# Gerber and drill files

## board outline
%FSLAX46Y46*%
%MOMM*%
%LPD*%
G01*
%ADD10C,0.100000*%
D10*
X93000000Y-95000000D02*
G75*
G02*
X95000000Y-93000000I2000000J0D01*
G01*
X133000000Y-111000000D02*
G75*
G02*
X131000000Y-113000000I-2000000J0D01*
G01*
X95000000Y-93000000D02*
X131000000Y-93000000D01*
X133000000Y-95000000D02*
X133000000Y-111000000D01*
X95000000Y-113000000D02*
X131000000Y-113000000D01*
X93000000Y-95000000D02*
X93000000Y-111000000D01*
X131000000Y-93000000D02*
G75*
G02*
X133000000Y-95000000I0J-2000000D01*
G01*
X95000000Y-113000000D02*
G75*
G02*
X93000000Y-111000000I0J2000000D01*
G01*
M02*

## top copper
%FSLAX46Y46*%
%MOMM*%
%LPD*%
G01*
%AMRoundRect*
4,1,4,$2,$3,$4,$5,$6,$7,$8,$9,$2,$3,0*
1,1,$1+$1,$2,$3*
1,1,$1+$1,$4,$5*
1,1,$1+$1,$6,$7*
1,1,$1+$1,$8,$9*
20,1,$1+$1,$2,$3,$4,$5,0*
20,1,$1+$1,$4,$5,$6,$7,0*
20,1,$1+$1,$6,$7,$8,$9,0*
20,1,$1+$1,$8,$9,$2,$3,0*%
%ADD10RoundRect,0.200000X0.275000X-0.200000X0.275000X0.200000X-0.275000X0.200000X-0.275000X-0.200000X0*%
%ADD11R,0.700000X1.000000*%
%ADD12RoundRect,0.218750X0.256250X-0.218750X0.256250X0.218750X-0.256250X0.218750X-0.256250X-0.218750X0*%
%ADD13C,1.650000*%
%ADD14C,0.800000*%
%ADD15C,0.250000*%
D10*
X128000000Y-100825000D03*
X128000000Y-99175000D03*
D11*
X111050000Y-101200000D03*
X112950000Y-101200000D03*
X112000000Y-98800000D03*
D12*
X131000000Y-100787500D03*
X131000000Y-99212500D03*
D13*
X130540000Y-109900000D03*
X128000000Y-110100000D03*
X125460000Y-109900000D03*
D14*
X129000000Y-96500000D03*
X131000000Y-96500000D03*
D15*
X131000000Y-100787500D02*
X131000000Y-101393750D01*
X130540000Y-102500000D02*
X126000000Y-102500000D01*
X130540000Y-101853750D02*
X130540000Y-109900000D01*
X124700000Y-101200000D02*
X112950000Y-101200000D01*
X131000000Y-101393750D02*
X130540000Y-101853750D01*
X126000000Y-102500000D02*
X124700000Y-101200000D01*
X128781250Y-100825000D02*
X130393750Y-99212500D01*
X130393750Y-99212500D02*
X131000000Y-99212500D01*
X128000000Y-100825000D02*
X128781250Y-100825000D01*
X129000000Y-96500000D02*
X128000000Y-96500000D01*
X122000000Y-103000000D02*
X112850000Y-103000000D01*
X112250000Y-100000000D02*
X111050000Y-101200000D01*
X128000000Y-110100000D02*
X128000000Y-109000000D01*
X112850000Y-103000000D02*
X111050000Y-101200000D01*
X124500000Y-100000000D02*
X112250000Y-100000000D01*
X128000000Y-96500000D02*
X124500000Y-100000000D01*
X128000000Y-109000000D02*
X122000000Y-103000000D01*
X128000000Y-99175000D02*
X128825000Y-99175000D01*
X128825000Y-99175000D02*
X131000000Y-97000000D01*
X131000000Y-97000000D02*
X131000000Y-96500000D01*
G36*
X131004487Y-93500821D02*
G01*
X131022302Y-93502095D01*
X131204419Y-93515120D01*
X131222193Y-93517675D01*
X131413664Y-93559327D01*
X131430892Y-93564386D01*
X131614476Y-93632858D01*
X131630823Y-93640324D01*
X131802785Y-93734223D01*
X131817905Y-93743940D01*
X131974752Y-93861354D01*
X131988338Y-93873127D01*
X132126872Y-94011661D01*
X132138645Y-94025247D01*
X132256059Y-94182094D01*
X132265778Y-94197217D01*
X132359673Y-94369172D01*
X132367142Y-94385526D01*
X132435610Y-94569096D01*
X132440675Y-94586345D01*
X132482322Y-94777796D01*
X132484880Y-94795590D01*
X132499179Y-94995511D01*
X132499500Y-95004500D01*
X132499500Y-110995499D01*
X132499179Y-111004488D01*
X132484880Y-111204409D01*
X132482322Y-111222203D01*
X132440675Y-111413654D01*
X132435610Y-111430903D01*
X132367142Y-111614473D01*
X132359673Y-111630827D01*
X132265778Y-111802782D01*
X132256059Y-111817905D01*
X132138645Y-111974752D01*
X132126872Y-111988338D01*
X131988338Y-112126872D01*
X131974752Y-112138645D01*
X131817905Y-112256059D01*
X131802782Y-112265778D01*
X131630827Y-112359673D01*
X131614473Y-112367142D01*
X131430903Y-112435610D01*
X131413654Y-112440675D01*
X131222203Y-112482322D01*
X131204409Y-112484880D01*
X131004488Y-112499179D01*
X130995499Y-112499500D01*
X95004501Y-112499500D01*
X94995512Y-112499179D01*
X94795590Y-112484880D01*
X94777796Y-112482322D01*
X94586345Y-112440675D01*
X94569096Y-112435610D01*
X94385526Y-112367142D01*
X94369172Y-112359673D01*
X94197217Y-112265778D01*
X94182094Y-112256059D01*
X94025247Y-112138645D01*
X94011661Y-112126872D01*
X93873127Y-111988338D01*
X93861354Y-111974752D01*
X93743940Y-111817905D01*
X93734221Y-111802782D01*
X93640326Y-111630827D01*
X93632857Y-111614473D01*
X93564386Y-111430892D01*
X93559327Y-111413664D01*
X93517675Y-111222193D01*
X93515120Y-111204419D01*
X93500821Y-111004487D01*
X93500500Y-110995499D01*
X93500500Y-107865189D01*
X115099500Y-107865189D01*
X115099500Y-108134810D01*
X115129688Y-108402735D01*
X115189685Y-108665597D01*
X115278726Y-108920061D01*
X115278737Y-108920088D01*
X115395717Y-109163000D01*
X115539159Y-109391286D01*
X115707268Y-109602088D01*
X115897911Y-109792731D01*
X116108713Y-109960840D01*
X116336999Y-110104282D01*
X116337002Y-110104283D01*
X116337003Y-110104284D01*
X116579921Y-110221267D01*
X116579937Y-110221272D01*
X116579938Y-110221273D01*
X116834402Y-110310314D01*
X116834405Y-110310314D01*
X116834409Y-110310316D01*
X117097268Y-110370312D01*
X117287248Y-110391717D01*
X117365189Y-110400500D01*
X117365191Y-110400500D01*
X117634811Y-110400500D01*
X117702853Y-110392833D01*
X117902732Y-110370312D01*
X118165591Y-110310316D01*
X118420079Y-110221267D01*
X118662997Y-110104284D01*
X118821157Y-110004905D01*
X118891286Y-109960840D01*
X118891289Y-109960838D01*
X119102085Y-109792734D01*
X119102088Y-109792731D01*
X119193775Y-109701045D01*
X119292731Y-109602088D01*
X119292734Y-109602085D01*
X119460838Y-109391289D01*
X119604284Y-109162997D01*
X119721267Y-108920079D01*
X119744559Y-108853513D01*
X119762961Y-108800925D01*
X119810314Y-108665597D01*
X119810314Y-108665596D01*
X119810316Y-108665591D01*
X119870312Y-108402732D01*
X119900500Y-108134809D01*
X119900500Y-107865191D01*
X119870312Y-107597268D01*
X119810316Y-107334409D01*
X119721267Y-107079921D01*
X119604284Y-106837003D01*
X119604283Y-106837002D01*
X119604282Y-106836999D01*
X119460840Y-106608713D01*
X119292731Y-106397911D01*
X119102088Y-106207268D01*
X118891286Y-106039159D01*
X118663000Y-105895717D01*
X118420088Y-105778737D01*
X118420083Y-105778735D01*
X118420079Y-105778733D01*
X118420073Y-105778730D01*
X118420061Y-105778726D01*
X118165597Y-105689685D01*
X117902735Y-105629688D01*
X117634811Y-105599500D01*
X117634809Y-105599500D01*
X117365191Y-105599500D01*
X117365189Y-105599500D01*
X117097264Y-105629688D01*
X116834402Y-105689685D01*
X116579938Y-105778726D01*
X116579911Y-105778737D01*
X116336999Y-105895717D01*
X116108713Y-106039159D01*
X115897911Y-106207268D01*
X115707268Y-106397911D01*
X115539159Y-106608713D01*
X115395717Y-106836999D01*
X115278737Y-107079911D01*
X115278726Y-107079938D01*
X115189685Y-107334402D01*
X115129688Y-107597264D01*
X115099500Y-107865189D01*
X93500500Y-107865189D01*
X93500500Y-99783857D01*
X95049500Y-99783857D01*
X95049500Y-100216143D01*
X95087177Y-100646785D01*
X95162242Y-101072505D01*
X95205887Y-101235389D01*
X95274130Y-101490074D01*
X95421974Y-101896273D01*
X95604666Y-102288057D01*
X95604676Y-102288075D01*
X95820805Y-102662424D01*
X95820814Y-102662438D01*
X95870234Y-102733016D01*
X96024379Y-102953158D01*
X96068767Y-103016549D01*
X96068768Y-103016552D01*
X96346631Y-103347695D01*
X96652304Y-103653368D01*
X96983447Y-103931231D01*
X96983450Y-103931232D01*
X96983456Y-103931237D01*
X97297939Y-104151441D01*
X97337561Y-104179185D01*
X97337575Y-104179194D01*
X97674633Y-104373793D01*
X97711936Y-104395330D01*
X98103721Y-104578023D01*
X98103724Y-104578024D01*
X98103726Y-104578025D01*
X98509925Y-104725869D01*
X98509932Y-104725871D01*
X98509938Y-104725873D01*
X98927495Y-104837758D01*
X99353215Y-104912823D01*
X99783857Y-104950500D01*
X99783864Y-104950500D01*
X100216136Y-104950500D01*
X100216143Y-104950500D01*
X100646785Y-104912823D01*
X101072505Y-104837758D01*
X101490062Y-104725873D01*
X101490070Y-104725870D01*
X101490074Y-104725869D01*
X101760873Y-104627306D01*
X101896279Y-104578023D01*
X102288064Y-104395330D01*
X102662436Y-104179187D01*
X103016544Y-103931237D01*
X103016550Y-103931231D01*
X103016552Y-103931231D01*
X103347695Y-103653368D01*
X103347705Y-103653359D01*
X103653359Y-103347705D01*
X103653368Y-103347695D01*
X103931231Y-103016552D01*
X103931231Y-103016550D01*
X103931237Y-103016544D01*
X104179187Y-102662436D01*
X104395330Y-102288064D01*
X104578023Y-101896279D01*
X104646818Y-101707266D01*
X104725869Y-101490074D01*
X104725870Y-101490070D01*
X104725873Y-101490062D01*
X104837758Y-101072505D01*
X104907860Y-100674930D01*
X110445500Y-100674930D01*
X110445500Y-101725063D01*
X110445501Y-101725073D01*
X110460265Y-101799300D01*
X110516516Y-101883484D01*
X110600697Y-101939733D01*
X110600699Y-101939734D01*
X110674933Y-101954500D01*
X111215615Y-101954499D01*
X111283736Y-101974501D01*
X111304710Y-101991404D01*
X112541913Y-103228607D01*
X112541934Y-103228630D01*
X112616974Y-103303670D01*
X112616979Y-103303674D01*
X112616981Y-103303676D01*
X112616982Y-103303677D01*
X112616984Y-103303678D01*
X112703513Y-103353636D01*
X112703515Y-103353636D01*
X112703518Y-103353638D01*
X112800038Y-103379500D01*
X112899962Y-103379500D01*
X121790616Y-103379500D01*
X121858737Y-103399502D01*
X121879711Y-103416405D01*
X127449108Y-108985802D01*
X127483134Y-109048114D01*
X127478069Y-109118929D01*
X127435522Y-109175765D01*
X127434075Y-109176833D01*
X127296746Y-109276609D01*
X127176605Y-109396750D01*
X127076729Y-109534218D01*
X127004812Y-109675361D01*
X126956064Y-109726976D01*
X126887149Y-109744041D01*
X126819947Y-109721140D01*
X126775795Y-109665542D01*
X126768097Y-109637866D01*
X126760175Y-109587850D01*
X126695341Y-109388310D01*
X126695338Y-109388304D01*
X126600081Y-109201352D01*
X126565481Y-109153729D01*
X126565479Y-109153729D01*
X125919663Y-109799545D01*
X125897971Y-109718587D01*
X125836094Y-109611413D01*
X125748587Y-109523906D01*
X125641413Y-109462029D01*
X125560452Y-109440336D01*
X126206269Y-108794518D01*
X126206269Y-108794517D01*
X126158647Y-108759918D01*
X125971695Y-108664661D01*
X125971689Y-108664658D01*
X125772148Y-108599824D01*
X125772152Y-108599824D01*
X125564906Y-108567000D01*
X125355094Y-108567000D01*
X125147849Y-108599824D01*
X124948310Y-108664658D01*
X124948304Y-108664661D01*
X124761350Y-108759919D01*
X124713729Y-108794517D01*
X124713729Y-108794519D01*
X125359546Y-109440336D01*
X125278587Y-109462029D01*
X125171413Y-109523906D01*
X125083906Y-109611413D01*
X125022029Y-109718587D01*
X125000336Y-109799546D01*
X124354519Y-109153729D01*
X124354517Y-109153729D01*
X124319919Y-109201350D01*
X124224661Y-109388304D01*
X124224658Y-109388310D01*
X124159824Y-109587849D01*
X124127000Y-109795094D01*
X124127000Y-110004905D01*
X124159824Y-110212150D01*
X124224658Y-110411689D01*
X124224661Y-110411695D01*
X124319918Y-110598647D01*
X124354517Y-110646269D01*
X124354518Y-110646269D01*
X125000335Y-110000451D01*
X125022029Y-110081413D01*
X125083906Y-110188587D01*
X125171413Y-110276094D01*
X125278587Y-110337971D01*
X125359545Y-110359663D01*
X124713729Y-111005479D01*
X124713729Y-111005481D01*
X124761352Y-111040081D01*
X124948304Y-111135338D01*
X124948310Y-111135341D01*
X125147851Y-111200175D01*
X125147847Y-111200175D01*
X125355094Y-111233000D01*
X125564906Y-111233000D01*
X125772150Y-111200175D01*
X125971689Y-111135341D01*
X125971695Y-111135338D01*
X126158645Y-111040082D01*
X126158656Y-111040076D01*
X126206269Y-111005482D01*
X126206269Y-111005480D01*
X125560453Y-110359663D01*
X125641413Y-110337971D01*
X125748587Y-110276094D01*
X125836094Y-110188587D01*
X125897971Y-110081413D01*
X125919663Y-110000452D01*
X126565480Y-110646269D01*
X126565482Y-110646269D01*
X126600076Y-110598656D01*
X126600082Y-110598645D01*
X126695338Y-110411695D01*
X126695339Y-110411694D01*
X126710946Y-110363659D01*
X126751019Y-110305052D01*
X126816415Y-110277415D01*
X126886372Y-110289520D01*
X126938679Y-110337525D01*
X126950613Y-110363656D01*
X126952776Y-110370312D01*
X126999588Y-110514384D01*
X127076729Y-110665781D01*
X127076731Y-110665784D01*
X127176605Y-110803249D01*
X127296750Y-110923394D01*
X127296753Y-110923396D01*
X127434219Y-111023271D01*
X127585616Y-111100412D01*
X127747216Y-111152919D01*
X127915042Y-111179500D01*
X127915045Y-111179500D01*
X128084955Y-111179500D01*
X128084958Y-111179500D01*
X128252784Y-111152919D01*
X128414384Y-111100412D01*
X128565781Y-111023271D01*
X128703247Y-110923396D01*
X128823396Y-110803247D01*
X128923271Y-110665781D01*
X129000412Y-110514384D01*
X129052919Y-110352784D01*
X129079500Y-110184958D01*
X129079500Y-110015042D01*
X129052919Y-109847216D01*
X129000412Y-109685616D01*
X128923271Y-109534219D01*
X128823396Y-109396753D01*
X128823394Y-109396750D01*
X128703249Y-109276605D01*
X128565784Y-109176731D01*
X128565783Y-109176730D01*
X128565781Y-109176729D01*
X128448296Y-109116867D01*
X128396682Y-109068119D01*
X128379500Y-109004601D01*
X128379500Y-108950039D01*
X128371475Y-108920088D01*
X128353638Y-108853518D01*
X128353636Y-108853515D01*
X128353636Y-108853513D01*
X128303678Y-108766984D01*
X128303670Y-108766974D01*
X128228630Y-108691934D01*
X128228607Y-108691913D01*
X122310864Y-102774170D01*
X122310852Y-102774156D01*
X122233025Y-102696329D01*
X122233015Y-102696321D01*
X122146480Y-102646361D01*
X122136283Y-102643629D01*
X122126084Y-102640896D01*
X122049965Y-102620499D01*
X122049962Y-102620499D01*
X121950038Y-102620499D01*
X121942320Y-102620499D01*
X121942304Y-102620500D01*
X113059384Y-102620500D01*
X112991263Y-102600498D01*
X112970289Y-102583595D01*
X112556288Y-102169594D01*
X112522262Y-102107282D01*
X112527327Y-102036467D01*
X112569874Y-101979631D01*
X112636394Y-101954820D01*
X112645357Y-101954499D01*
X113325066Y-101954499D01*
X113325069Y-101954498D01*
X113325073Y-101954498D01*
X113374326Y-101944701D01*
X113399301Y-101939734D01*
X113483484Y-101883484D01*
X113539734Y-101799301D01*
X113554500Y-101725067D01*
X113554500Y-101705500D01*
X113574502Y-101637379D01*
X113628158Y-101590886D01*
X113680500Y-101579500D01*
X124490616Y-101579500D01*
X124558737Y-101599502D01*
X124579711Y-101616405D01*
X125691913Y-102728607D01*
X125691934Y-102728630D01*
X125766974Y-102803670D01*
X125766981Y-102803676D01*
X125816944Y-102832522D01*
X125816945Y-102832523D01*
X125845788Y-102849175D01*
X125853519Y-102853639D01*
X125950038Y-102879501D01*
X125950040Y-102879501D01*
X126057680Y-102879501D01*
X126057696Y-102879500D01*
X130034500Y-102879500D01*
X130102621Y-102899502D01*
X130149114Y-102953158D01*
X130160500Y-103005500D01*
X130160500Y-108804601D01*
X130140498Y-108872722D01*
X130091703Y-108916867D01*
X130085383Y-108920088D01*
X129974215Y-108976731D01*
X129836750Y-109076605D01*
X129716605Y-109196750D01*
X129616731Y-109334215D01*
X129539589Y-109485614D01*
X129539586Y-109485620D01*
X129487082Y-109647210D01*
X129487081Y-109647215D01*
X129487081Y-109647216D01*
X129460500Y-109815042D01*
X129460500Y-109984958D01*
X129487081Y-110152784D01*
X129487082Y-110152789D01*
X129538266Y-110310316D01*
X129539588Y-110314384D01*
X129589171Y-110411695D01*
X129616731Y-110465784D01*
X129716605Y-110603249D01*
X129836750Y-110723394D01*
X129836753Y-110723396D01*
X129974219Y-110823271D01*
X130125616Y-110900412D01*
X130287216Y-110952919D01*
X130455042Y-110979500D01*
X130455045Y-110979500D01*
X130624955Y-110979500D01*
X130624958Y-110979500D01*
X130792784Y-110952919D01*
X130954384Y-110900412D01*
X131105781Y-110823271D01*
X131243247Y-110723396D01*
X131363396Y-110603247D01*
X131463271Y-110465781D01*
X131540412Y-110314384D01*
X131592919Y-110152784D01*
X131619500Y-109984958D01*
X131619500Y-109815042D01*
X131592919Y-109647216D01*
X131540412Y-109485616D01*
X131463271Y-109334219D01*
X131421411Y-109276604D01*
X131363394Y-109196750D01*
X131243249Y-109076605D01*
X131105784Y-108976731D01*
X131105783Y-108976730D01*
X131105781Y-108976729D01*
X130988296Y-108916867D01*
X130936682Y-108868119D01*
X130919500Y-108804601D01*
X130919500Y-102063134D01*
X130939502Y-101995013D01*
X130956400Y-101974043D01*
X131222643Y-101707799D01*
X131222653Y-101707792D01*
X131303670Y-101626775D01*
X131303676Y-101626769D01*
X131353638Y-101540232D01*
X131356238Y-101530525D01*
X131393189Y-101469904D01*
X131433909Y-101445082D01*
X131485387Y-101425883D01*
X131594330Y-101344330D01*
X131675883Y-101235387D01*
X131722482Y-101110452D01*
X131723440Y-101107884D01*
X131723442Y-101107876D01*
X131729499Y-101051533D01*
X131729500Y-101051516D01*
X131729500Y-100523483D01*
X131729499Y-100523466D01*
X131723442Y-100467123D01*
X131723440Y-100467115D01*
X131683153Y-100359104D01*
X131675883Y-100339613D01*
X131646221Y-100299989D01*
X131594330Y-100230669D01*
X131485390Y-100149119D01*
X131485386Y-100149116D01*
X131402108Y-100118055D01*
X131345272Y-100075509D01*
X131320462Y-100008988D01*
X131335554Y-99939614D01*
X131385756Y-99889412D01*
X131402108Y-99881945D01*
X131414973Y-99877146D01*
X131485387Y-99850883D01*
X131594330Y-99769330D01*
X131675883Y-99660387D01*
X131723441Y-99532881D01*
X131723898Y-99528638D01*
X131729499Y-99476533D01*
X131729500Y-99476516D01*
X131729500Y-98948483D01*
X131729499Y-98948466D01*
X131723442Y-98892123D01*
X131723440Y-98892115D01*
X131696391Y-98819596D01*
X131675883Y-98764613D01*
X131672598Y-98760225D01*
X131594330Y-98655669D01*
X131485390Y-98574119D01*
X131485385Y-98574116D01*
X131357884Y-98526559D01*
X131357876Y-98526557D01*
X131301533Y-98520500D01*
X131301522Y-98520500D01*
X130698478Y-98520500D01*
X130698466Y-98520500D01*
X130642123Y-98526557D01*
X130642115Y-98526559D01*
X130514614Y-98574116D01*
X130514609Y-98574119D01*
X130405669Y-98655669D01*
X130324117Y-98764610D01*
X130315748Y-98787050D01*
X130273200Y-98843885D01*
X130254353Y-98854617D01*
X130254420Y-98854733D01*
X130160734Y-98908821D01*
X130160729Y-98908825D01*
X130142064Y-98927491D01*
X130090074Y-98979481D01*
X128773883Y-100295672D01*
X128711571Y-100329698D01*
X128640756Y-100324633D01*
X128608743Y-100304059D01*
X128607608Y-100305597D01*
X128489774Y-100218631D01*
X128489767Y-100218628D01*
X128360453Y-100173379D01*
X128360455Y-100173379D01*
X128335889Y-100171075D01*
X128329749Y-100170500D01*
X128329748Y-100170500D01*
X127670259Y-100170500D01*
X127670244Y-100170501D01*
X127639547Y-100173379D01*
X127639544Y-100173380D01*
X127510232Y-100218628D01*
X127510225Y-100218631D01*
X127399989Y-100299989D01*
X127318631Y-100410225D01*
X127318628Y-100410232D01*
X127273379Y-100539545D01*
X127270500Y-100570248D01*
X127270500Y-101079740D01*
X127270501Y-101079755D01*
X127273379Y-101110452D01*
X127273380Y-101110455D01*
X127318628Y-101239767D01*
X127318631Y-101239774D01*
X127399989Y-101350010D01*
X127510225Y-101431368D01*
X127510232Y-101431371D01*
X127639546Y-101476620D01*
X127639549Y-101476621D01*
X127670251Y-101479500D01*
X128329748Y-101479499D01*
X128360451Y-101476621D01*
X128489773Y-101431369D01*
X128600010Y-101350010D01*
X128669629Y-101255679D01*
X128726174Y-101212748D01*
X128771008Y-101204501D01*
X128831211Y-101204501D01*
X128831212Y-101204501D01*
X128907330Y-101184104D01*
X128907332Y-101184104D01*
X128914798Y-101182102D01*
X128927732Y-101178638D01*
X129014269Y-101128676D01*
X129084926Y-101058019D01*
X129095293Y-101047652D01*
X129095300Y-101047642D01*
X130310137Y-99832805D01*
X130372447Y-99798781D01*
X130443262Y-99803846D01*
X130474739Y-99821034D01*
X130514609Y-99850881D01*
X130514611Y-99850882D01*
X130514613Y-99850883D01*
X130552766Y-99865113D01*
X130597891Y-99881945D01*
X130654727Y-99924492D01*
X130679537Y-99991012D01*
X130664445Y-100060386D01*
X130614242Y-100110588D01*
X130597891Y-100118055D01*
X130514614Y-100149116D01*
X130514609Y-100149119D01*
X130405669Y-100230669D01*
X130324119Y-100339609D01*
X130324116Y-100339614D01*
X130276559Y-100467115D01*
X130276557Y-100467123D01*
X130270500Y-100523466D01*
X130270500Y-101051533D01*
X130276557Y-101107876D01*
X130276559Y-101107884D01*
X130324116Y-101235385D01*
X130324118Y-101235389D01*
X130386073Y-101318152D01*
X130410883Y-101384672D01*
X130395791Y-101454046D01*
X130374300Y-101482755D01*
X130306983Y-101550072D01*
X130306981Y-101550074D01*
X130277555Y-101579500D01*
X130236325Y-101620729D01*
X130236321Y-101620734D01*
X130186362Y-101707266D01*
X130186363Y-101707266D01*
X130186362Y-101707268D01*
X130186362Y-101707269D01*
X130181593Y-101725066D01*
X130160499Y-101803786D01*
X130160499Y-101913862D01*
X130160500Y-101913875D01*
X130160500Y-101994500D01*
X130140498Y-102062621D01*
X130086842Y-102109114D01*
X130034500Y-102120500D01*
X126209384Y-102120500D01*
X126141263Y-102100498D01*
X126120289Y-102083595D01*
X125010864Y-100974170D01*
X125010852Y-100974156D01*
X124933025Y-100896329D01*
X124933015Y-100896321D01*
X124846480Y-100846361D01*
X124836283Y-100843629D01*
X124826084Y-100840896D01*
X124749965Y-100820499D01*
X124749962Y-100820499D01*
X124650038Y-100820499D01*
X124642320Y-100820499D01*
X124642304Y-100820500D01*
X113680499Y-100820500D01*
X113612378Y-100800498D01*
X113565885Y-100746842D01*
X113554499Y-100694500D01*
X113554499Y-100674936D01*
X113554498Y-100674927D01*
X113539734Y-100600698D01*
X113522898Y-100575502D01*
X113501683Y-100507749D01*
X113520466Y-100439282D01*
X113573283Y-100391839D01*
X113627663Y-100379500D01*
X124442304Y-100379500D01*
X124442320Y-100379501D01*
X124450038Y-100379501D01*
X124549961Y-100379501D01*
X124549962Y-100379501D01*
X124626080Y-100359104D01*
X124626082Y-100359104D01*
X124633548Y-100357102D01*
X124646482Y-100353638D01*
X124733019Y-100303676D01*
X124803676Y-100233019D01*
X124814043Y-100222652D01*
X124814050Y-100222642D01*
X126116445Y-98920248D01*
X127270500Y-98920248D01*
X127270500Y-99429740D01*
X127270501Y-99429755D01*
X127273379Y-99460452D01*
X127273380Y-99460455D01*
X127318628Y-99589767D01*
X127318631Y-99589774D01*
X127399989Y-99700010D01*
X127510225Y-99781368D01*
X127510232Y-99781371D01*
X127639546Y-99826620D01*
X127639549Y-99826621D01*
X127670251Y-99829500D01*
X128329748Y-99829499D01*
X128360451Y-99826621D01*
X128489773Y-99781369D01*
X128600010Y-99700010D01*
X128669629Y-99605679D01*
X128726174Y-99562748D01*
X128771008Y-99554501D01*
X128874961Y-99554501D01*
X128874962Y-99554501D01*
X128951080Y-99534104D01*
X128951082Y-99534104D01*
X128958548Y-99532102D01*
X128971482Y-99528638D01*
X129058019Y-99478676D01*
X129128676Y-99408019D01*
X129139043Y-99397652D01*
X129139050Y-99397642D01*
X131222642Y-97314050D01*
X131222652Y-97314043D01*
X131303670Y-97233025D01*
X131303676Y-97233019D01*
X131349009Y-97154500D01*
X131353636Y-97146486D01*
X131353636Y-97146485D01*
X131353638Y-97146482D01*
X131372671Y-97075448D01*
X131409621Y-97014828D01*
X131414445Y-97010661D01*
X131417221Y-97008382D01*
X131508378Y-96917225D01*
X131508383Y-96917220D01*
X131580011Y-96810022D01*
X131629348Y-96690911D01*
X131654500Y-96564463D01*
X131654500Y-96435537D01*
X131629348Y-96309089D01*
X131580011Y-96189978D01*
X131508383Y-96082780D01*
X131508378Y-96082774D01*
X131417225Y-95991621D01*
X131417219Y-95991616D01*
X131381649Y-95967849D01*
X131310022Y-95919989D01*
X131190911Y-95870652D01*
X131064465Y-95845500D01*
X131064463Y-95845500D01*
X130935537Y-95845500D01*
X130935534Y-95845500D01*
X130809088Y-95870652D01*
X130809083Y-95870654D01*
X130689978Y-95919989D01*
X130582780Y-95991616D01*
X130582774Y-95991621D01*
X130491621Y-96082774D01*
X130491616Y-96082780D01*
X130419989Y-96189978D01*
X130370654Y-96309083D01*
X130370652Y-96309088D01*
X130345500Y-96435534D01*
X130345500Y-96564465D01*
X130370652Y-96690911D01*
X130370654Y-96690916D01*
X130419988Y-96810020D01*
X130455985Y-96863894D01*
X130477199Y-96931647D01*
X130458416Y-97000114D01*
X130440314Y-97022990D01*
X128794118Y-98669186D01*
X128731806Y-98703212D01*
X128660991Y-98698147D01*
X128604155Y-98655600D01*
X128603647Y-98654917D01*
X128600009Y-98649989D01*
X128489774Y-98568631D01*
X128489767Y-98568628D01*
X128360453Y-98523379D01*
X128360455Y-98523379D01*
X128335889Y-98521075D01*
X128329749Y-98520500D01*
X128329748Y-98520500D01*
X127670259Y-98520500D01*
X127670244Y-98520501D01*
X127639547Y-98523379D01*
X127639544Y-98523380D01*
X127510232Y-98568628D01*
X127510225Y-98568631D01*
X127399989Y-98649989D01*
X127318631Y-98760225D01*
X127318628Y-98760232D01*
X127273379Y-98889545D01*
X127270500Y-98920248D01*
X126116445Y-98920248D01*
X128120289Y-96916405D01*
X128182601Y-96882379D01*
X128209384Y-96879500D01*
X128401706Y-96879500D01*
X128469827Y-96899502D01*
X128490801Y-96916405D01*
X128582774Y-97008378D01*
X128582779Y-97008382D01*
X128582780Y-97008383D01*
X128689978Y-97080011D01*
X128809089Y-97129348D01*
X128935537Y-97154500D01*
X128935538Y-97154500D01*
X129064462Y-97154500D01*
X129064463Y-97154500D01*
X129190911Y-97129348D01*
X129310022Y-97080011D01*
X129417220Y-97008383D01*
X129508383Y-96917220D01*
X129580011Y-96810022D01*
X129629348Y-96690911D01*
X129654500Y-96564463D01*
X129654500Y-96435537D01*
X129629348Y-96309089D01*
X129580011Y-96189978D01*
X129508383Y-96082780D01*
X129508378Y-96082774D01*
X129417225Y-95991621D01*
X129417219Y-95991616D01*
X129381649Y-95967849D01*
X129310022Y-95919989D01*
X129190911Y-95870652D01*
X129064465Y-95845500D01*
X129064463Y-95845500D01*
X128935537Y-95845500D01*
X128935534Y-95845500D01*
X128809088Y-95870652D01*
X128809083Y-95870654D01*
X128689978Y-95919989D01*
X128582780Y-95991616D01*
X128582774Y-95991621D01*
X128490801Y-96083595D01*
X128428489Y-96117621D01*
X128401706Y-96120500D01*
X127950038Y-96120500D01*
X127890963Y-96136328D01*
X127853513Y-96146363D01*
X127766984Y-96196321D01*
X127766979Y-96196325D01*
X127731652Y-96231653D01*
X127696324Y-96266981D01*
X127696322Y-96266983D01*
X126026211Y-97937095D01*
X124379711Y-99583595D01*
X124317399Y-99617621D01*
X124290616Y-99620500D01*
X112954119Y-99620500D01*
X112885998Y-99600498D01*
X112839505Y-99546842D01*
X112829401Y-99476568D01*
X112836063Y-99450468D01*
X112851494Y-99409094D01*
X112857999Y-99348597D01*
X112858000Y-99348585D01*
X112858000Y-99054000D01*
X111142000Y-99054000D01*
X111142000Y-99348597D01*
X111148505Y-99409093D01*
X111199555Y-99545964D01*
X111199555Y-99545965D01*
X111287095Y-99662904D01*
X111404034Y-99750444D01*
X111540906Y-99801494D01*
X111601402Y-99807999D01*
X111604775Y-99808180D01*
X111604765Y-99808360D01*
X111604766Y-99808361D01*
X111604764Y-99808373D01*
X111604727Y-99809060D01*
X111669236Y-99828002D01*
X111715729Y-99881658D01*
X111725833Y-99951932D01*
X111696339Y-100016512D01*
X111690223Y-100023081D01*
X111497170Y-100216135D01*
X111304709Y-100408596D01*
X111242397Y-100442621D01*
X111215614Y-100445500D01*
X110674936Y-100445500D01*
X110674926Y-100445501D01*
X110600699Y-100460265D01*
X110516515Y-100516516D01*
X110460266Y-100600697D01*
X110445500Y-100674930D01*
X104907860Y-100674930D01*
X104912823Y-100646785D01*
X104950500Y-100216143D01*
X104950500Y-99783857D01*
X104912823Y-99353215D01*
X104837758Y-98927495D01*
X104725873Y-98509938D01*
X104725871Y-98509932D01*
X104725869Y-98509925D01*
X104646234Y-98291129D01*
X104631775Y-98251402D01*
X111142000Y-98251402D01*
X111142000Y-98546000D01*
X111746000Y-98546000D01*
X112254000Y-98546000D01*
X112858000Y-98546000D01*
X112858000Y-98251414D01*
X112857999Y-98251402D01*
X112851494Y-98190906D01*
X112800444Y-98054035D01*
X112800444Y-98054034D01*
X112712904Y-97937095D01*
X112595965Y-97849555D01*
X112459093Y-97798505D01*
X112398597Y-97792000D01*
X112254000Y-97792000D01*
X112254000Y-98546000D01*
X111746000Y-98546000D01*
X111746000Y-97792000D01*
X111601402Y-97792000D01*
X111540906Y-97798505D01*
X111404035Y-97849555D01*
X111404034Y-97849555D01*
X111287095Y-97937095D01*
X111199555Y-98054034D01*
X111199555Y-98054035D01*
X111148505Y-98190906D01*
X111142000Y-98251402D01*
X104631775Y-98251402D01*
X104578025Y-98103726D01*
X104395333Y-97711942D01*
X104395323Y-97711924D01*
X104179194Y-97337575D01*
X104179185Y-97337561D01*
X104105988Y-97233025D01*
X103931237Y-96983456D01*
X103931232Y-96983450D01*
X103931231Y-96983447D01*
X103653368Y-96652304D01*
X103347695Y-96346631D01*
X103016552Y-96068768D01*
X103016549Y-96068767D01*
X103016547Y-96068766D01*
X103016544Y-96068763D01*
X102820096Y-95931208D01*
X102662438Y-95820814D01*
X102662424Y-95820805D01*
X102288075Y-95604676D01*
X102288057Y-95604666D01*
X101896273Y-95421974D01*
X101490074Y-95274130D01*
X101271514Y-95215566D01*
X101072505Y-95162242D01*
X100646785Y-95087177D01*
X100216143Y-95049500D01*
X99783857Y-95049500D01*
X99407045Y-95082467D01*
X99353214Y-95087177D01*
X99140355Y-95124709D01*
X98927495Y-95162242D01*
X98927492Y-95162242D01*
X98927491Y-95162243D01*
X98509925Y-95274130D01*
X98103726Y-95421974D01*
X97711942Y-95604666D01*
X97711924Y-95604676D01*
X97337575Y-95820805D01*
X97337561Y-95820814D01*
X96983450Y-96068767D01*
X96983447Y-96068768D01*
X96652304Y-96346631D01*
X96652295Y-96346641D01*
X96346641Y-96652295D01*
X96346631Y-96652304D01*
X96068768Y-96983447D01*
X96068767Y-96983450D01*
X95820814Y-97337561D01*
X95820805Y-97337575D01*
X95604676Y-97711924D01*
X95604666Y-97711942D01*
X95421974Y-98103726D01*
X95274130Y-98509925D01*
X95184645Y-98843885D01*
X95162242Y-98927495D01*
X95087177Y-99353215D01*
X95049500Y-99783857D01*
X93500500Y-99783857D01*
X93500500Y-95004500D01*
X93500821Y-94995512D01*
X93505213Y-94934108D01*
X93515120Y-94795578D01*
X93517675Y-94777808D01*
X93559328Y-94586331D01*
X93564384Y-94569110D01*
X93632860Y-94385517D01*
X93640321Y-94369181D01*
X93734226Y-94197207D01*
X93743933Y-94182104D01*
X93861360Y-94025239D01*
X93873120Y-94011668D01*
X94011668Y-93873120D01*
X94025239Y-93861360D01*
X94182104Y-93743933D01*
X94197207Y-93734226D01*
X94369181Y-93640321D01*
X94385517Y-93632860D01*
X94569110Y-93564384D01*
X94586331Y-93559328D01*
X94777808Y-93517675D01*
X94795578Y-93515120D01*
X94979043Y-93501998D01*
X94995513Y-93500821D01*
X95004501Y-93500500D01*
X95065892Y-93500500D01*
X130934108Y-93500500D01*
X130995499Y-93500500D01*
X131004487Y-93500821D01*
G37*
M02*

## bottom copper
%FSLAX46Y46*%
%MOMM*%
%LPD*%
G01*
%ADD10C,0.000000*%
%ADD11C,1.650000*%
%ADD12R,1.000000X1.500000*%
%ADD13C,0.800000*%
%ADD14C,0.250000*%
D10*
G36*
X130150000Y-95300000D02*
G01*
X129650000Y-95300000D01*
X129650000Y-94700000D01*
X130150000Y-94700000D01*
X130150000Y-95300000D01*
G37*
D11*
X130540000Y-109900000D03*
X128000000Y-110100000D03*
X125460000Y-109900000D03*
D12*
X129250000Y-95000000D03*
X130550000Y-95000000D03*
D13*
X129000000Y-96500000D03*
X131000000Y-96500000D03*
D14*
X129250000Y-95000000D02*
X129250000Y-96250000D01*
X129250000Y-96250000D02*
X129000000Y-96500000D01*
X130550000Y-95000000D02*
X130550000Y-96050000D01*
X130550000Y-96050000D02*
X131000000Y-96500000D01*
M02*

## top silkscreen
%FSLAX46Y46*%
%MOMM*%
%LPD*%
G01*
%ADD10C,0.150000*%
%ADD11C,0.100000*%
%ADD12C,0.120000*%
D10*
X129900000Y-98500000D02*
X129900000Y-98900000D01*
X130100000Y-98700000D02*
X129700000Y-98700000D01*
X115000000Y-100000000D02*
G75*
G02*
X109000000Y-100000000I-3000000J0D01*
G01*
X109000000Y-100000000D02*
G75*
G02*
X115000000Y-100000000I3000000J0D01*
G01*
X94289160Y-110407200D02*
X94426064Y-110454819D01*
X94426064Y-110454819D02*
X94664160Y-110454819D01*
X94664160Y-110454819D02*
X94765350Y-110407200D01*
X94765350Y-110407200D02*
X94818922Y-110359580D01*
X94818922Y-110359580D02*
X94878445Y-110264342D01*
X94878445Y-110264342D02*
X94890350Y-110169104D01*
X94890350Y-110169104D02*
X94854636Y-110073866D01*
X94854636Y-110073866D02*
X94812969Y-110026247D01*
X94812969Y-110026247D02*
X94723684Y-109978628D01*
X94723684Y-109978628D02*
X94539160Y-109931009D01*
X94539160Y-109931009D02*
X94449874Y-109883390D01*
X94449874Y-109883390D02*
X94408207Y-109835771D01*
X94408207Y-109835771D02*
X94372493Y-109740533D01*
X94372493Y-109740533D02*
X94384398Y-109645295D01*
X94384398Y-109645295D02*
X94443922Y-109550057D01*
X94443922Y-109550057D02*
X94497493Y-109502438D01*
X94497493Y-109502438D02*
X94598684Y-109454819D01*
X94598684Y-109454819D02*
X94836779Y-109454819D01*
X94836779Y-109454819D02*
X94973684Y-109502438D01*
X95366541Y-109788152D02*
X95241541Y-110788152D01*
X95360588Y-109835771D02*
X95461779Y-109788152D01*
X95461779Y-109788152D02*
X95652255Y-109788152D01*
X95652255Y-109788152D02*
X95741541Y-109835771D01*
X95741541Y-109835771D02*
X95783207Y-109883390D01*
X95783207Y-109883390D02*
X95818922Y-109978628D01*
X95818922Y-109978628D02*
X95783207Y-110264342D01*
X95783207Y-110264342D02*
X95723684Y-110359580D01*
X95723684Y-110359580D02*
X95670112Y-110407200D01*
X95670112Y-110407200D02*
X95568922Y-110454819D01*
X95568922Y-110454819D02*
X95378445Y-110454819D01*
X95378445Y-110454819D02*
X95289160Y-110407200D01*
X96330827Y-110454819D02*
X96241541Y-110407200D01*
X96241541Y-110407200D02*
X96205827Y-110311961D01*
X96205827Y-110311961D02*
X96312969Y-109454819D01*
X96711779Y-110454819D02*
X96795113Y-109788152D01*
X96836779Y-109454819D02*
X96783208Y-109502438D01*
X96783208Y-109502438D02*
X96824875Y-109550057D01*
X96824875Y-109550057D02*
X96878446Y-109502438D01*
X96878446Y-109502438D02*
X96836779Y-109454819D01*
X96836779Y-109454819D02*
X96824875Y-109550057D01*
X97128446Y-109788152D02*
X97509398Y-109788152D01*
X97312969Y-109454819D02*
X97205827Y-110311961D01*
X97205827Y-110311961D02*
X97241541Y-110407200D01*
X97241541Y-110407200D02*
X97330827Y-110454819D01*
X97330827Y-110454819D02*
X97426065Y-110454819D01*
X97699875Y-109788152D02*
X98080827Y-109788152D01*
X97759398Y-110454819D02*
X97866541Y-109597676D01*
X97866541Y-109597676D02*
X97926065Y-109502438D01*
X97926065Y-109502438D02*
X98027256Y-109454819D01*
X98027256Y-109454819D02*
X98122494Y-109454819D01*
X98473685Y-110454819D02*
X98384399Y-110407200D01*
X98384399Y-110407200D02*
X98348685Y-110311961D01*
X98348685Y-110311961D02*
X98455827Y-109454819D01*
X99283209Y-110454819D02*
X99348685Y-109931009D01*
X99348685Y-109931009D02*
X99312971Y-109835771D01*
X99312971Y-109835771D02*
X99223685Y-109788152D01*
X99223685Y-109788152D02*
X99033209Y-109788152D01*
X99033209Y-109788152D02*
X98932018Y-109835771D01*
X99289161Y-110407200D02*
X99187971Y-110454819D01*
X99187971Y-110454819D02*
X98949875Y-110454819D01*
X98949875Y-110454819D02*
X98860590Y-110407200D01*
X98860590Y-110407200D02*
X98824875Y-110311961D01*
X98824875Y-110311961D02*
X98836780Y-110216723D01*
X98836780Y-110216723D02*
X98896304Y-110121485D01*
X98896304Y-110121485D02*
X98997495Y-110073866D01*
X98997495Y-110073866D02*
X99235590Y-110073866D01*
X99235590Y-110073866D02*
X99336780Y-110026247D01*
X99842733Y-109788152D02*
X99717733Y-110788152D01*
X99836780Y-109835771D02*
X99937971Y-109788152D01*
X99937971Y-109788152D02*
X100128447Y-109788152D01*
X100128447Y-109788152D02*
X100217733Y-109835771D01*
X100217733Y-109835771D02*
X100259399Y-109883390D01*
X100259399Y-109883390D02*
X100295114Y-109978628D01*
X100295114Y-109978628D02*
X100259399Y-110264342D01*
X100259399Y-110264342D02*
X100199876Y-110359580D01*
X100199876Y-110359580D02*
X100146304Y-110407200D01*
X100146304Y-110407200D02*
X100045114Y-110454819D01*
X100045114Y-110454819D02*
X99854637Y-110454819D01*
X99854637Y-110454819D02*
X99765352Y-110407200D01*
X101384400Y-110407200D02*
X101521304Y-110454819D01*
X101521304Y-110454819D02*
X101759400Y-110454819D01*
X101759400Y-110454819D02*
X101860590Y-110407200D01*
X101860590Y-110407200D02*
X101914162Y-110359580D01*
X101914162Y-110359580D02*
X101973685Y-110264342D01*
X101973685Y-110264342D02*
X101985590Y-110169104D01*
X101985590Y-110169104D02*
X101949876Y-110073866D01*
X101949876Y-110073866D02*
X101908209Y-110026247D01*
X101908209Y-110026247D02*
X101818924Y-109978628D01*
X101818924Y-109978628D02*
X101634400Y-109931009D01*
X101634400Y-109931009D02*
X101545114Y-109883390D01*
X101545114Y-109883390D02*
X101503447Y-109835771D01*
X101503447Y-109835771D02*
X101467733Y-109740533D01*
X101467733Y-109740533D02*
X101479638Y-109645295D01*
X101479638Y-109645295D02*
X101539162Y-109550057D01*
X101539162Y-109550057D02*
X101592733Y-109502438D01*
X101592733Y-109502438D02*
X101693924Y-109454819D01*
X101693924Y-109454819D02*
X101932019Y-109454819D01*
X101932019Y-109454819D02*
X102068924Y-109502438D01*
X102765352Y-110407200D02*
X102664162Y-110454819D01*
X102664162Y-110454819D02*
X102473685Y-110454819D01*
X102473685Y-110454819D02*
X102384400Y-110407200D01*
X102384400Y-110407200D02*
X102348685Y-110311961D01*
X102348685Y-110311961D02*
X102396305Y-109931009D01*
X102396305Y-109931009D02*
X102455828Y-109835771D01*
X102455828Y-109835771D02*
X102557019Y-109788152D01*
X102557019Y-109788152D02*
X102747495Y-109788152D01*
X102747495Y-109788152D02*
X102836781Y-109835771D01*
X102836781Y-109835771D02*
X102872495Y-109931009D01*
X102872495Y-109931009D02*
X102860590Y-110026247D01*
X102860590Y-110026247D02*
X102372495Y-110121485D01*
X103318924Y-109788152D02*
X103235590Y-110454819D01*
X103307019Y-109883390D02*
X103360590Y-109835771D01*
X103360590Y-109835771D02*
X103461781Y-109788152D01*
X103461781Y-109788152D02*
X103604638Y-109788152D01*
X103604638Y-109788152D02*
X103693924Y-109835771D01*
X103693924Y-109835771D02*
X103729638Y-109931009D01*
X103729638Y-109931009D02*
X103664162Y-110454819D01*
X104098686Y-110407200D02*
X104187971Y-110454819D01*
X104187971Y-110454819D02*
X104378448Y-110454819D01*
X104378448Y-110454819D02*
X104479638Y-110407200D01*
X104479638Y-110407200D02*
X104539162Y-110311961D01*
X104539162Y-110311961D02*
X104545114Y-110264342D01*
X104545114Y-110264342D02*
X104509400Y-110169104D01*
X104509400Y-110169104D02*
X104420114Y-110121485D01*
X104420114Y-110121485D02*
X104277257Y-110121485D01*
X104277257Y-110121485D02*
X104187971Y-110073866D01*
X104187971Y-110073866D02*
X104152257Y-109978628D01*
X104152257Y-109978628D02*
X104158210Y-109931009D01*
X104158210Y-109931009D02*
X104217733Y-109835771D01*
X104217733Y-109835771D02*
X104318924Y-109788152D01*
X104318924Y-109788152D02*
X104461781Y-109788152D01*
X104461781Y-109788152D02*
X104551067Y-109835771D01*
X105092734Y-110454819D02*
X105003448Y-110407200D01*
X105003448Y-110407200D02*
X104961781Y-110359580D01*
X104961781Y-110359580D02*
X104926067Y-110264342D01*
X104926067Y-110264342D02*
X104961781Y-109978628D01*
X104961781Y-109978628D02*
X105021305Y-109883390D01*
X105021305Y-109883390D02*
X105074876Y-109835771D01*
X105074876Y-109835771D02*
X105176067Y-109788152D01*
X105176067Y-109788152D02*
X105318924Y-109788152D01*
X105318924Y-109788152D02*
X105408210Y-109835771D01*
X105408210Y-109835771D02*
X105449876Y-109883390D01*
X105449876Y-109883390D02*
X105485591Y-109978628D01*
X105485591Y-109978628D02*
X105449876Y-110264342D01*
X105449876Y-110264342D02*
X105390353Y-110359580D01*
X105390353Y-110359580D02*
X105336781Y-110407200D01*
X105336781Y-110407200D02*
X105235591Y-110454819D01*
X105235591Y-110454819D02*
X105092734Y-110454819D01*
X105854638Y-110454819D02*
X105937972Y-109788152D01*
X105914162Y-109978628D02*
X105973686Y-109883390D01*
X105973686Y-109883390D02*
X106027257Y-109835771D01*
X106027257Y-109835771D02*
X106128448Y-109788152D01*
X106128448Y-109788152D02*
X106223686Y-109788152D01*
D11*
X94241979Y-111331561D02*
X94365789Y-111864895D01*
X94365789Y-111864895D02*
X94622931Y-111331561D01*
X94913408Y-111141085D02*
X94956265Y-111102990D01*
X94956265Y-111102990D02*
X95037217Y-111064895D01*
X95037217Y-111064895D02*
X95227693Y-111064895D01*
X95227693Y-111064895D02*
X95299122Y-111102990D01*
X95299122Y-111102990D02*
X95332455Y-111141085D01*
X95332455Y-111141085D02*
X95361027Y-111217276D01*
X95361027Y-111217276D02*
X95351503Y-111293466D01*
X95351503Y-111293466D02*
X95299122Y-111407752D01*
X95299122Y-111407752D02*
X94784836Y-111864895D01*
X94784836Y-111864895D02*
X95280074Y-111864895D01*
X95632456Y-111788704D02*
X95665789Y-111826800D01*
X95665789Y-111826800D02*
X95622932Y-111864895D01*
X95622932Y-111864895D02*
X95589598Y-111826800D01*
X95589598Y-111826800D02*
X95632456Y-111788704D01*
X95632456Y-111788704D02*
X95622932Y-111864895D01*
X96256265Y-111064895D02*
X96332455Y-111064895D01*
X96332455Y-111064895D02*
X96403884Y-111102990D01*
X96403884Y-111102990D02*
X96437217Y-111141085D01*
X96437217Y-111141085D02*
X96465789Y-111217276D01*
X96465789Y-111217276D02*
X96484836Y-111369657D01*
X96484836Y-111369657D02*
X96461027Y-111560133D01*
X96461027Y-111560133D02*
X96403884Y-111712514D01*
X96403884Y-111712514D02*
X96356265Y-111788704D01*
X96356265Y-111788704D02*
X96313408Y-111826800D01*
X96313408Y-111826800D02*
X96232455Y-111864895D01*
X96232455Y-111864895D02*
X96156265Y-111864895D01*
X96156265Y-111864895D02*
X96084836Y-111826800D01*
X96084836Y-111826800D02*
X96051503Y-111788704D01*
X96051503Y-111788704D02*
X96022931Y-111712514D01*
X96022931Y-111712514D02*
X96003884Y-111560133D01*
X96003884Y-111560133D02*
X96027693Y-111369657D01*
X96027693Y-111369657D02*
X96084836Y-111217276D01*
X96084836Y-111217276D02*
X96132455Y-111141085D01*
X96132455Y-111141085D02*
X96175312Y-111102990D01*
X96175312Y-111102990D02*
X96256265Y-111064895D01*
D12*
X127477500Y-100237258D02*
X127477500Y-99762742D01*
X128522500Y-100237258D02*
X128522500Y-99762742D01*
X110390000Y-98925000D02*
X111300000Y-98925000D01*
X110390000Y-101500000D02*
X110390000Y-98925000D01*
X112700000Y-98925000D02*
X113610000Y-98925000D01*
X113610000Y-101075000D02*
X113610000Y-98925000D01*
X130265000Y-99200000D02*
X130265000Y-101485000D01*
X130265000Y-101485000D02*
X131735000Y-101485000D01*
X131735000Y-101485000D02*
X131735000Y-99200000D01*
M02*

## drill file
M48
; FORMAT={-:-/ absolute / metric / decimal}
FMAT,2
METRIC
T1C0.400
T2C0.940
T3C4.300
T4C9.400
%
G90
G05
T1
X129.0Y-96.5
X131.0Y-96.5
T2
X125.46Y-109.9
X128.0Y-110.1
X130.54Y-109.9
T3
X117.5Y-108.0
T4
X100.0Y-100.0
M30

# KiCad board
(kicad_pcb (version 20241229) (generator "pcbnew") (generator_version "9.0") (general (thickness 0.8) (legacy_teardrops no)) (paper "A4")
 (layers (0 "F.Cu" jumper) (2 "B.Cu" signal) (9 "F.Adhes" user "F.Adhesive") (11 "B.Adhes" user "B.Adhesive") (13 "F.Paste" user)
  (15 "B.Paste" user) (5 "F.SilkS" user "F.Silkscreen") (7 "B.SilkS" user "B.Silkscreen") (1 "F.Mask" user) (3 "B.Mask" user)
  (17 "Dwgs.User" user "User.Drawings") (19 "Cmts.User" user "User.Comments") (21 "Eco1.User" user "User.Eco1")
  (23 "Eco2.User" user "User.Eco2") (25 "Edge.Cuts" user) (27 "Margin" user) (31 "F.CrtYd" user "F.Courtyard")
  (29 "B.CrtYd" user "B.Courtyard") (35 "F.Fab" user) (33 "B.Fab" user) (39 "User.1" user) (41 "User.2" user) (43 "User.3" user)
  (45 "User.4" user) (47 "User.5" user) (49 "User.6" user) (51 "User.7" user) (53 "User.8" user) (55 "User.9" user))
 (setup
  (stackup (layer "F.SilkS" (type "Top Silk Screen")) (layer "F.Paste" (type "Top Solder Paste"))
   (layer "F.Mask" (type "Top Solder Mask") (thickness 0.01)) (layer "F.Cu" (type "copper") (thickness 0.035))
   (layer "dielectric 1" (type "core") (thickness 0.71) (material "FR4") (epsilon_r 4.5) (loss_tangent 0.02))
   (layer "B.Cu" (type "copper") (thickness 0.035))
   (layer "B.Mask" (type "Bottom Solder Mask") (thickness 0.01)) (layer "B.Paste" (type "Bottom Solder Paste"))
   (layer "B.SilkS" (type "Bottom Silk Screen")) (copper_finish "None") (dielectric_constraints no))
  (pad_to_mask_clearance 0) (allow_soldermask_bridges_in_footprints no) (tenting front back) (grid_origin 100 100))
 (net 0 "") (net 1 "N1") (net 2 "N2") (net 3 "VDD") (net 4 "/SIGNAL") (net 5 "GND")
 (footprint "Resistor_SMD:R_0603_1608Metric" (layer "F.Cu") (at 128 100 90)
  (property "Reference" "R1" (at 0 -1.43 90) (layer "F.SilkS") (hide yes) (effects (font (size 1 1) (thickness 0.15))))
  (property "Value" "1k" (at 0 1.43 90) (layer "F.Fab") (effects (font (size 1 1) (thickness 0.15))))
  (fp_line (start -0.237258 -0.5225) (end 0.237258 -0.5225) (stroke (width 0.12) (type solid)) (layer "F.SilkS"))
  (fp_line (start -0.237258 0.5225) (end 0.237258 0.5225) (stroke (width 0.12) (type solid)) (layer "F.SilkS"))
  (pad "1" smd roundrect (at -0.825 0 90) (size 0.8 0.95) (layers "F.Cu" "F.Mask" "F.Paste") (roundrect_rratio 0.25) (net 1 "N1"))
  (pad "2" smd roundrect (at 0.825 0 90) (size 0.8 0.95) (layers "F.Cu" "F.Mask" "F.Paste") (roundrect_rratio 0.25) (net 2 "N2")))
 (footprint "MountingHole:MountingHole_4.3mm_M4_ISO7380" (layer "F.Cu") (at 117.5 108)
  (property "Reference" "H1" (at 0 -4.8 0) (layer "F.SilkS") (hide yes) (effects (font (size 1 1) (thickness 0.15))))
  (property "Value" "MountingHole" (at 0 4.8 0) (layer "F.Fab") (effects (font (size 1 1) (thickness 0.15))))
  (pad "" np_thru_hole circle (at 0 0) (size 4.3 4.3) (drill 4.3) (layers "*.Cu" "*.Mask")))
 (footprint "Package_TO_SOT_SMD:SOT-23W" (layer "F.Cu") (at 112 100 90)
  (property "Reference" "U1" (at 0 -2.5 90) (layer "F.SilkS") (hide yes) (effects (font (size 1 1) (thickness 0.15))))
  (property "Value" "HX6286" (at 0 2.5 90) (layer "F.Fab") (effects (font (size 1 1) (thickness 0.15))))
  (fp_line (start 1.075 -1.61) (end 1.075 -0.7) (stroke (width 0.12) (type solid)) (layer "F.SilkS"))
  (fp_line (start -1.5 -1.61) (end 1.075 -1.61) (stroke (width 0.12) (type solid)) (layer "F.SilkS"))
  (fp_line (start 1.075 0.7) (end 1.075 1.61) (stroke (width 0.12) (type solid)) (layer "F.SilkS"))
  (fp_line (start -1.075 1.61) (end 1.075 1.61) (stroke (width 0.12) (type solid)) (layer "F.SilkS"))
  (pad "1" smd rect (at -1.2 -0.95 90) (size 1 0.7) (layers "F.Cu" "F.Mask" "F.Paste") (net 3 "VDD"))
  (pad "2" smd rect (at -1.2 0.95 90) (size 1 0.7) (layers "F.Cu" "F.Mask" "F.Paste") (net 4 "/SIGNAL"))
  (pad "3" smd rect (at 1.2 0 90) (size 1 0.7) (layers "F.Cu" "F.Mask" "F.Paste") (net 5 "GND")))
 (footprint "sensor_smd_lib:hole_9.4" (layer "F.Cu") (at 100 100)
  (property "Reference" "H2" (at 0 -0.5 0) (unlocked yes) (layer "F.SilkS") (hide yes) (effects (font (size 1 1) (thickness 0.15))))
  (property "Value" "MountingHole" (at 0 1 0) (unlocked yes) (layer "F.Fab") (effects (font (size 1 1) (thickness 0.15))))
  (pad "" np_thru_hole circle (at 0 0) (size 9.4 9.4) (drill 9.4) (layers "*.Cu" "*.Mask")))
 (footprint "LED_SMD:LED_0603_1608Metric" (layer "F.Cu") (at 131 100 90)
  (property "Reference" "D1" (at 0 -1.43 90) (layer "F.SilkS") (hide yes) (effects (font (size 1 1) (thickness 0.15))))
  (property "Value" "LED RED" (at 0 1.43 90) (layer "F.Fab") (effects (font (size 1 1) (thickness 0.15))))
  (fp_line (start 0.8 -0.735) (end -1.485 -0.735) (stroke (width 0.12) (type solid)) (layer "F.SilkS"))
  (fp_line (start -1.485 -0.735) (end -1.485 0.735) (stroke (width 0.12) (type solid)) (layer "F.SilkS"))
  (fp_line (start -1.485 0.735) (end 0.8 0.735) (stroke (width 0.12) (type solid)) (layer "F.SilkS"))
  (pad "1" smd roundrect (at -0.7875 0 90) (size 0.875 0.95) (layers "F.Cu" "F.Mask" "F.Paste") (roundrect_rratio 0.25) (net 4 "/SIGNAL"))
  (pad "2" smd roundrect (at 0.7875 0 90) (size 0.875 0.95) (layers "F.Cu" "F.Mask" "F.Paste") (roundrect_rratio 0.25) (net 1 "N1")))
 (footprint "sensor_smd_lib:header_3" (layer "B.Cu") (at 128 113 180)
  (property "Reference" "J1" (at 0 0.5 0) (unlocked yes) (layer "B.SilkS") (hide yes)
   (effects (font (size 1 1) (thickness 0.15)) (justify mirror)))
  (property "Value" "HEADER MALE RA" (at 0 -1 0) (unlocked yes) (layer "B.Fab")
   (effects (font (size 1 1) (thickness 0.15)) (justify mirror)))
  (pad "1" thru_hole circle (at -2.54 3.1 180) (size 1.65 1.65) (drill 0.94) (layers "*.Cu" "*.Mask") (remove_unused_layers no)
   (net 4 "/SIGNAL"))
  (pad "2" thru_hole circle (at 0 2.9 180) (size 1.65 1.65) (drill 0.94) (layers "*.Cu" "*.Mask") (remove_unused_layers no) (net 3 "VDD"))
  (pad "3" thru_hole circle (at 2.54 3.1 180) (size 1.65 1.65) (drill 0.94) (layers "*.Cu" "*.Mask") (remove_unused_layers no) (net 5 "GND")))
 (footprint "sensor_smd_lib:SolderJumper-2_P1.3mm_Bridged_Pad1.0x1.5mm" (layer "B.Cu") (at 129.9 95)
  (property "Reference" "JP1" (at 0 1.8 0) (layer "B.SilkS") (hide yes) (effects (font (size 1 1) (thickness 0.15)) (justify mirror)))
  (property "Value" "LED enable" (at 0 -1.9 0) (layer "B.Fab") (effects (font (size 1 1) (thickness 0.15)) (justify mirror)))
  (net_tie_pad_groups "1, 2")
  (fp_poly (pts (xy -0.25 0.3) (xy 0.25 0.3) (xy 0.25 -0.3) (xy -0.25 -0.3)) (stroke (width 0) (type solid)) (fill yes) (layer "B.Cu"))
  (pad "1" smd rect (at -0.65 0) (size 1 1.5) (layers "B.Cu" "B.Mask") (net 3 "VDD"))
  (pad "2" smd rect (at 0.65 0) (size 1 1.5) (layers "B.Cu" "B.Mask") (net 2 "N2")))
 (gr_line (start 129.9 98.5) (end 129.9 98.9) (stroke (width 0.15) (type solid)) (layer "F.SilkS"))
 (gr_line (start 130.1 98.7) (end 129.7 98.7) (stroke (width 0.15) (type solid)) (layer "F.SilkS"))
 (gr_circle (center 112 100) (end 115 100) (stroke (width 0.15) (type solid)) (fill no) (layer "F.SilkS"))
 (gr_arc (start 93 95) (mid 93.585786 93.585786) (end 95 93) (stroke (width 0.1) (type solid)) (layer "Edge.Cuts"))
 (gr_arc (start 133 111) (mid 132.414214 112.414214) (end 131 113) (stroke (width 0.1) (type solid)) (layer "Edge.Cuts"))
 (gr_line (start 95 93) (end 131 93) (stroke (width 0.1) (type solid)) (layer "Edge.Cuts"))
 (gr_line (start 133 95) (end 133 111) (stroke (width 0.1) (type solid)) (layer "Edge.Cuts"))
 (gr_line (start 95 113) (end 131 113) (stroke (width 0.1) (type solid)) (layer "Edge.Cuts"))
 (gr_line (start 93 95) (end 93 111) (stroke (width 0.1) (type solid)) (layer "Edge.Cuts"))
 (gr_arc (start 131 93) (mid 132.414214 93.585786) (end 133 95) (stroke (width 0.1) (type solid)) (layer "Edge.Cuts"))
 (gr_arc (start 95 113) (mid 93.585786 112.414214) (end 93 111) (stroke (width 0.1) (type solid)) (layer "Edge.Cuts"))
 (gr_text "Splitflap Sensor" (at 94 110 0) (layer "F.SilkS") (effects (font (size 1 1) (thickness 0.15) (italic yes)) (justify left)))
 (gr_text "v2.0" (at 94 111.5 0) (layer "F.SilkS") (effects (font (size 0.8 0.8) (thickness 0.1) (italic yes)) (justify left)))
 (segment (start 131 100.7875) (end 131 101.39375) (width 0.25) (layer "F.Cu") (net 4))
 (segment (start 130.54 102.5) (end 126 102.5) (width 0.25) (layer "F.Cu") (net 4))
 (segment (start 130.54 101.85375) (end 130.54 109.9) (width 0.25) (layer "F.Cu") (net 4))
 (segment (start 124.7 101.2) (end 112.95 101.2) (width 0.25) (layer "F.Cu") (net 4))
 (segment (start 131 101.39375) (end 130.54 101.85375) (width 0.25) (layer "F.Cu") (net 4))
 (segment (start 126 102.5) (end 124.7 101.2) (width 0.25) (layer "F.Cu") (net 4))
 (segment (start 128.78125 100.825) (end 130.39375 99.2125) (width 0.25) (layer "F.Cu") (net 1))
 (segment (start 130.39375 99.2125) (end 131 99.2125) (width 0.25) (layer "F.Cu") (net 1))
 (segment (start 128 100.825) (end 128.78125 100.825) (width 0.25) (layer "F.Cu") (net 1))
 (segment (start 129 96.5) (end 128 96.5) (width 0.25) (layer "F.Cu") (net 3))
 (segment (start 122 103) (end 112.85 103) (width 0.25) (layer "F.Cu") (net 3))
 (segment (start 112.25 100) (end 111.05 101.2) (width 0.25) (layer "F.Cu") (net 3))
 (segment (start 128 110.1) (end 128 109) (width 0.25) (layer "F.Cu") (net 3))
 (segment (start 112.85 103) (end 111.05 101.2) (width 0.25) (layer "F.Cu") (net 3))
 (segment (start 124.5 100) (end 112.25 100) (width 0.25) (layer "F.Cu") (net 3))
 (segment (start 128 96.5) (end 124.5 100) (width 0.25) (layer "F.Cu") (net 3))
 (segment (start 128 109) (end 122 103) (width 0.25) (layer "F.Cu") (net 3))
 (via (at 129 96.5) (size 0.8) (drill 0.4) (layers "F.Cu" "B.Cu") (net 3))
 (segment (start 129.25 95) (end 129.25 96.25) (width 0.25) (layer "B.Cu") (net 3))
 (segment (start 129.25 96.25) (end 129 96.5) (width 0.25) (layer "B.Cu") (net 3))
 (segment (start 128 99.175) (end 128.825 99.175) (width 0.25) (layer "F.Cu") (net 2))
 (segment (start 128.825 99.175) (end 131 97) (width 0.25) (layer "F.Cu") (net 2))
 (segment (start 131 97) (end 131 96.5) (width 0.25) (layer "F.Cu") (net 2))
 (via (at 131 96.5) (size 0.8) (drill 0.4) (layers "F.Cu" "B.Cu") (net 2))
 (segment (start 130.55 95) (end 130.55 96.05) (width 0.25) (layer "B.Cu") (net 2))
 (segment (start 130.55 96.05) (end 131 96.5) (width 0.25) (layer "B.Cu") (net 2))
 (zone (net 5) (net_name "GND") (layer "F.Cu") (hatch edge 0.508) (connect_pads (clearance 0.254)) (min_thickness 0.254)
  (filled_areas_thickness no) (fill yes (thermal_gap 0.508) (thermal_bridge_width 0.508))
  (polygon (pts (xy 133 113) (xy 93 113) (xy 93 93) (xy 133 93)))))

